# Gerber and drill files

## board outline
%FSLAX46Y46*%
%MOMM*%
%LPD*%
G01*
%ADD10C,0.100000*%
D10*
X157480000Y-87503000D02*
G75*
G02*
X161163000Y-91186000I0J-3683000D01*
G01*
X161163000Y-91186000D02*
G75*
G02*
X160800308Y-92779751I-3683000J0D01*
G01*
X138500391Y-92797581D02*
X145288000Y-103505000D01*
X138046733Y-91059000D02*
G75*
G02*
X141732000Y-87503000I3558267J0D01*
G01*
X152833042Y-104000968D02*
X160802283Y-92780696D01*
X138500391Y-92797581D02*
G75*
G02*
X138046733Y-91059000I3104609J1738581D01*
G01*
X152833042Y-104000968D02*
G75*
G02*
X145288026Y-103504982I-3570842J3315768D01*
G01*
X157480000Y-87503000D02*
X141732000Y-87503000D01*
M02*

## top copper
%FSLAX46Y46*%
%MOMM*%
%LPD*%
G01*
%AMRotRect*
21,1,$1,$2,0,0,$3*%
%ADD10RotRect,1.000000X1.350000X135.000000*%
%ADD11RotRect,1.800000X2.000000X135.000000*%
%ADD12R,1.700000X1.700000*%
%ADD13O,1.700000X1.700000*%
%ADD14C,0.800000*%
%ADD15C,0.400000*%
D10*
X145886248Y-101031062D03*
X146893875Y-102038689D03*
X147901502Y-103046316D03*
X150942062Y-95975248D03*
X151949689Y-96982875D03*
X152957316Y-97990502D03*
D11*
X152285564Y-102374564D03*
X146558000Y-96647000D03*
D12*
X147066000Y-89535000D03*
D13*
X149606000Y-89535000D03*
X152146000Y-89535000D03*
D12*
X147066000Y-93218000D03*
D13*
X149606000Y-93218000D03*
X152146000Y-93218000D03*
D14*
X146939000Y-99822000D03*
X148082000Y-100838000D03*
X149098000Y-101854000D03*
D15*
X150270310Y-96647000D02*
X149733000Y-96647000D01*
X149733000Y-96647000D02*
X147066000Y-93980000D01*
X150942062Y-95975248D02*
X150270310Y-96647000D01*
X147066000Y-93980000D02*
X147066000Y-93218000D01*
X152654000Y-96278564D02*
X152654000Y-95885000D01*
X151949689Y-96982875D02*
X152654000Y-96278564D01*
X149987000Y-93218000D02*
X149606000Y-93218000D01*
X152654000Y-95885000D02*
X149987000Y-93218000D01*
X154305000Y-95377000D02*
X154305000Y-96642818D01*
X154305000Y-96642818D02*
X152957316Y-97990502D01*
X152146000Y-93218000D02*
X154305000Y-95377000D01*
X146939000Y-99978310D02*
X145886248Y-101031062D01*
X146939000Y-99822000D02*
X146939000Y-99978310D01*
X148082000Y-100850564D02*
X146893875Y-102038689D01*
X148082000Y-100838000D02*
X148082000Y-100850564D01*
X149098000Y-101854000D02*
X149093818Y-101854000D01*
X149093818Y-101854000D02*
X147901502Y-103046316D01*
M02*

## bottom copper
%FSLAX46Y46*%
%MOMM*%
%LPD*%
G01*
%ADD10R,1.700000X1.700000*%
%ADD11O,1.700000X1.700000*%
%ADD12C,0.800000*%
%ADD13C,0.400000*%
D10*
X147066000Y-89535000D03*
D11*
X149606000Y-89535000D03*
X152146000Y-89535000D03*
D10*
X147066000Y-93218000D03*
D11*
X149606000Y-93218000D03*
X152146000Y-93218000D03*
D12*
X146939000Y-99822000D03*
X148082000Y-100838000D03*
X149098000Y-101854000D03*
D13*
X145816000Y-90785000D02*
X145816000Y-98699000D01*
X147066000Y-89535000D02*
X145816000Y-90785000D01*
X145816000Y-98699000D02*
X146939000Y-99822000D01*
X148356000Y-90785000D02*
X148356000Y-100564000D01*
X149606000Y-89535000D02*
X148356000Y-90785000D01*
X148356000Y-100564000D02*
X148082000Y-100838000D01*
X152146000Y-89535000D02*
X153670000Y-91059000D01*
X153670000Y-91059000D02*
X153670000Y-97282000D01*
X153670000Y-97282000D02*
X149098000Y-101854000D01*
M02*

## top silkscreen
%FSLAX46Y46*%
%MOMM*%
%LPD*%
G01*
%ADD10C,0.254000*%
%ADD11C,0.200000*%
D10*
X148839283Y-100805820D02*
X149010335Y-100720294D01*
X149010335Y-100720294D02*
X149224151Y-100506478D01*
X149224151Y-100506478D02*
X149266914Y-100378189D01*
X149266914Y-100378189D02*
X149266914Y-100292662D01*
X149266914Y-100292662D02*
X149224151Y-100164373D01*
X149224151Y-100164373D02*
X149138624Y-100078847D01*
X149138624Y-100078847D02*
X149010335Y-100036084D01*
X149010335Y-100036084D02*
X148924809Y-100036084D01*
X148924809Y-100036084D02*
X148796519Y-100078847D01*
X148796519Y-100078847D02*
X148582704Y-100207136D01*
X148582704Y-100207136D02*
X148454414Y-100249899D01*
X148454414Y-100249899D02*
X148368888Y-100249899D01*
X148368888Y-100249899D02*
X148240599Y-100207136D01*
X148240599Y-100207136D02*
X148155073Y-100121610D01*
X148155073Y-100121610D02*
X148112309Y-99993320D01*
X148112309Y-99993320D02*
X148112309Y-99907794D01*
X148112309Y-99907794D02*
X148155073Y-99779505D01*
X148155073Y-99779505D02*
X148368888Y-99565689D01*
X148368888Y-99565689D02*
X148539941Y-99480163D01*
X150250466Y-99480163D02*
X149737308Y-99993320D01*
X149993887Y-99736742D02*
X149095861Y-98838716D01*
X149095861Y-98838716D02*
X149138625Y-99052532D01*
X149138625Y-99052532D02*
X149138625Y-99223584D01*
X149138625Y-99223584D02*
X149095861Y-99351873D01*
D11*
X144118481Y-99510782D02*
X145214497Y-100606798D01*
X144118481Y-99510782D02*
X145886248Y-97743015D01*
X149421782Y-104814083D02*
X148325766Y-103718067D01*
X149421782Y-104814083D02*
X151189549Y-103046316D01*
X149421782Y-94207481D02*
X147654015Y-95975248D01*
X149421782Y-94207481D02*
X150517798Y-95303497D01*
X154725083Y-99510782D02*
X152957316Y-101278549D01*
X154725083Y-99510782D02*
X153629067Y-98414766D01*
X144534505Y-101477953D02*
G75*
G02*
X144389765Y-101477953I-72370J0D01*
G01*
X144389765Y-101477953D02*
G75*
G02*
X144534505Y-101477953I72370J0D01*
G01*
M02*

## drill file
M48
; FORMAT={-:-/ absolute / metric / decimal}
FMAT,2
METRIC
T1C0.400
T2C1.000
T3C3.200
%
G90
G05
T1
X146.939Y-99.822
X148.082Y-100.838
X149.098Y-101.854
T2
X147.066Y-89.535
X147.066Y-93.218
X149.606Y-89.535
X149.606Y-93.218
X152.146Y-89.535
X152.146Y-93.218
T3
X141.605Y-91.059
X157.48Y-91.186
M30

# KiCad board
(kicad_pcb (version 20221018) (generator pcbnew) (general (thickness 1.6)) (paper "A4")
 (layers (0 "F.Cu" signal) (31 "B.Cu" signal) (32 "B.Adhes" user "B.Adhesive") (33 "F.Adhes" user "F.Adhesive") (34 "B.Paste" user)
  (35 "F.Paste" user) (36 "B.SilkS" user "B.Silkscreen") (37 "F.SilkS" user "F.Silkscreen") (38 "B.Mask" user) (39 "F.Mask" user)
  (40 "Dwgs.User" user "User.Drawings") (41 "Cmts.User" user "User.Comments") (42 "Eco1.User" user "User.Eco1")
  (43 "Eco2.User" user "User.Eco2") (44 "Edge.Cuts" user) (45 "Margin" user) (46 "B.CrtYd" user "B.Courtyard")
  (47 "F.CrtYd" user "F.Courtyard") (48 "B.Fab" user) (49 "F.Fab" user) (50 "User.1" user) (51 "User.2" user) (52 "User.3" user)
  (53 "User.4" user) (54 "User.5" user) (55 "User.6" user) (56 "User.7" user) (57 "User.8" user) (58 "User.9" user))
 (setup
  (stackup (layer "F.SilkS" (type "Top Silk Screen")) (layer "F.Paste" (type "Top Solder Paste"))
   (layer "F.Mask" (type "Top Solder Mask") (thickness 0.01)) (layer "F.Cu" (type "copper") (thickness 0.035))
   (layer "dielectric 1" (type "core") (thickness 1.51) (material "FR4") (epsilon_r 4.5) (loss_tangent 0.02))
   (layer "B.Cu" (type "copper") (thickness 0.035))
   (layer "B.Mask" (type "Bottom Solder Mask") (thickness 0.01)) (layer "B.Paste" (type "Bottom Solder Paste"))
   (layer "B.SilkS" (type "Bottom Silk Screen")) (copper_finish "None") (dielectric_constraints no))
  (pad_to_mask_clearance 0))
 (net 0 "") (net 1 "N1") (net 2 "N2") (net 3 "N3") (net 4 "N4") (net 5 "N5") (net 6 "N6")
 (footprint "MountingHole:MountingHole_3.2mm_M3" (layer "F.Cu") (at 141.605 91.059)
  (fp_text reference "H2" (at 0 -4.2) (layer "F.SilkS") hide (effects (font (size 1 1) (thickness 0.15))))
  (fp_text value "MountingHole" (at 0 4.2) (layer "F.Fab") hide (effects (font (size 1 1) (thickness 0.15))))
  (pad "" np_thru_hole circle (at 0 0) (size 3.2 3.2) (drill 3.2) (layers "*.Cu" "*.Mask")))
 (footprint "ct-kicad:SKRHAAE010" (layer "F.Cu") (at 149.421782 99.510782 45)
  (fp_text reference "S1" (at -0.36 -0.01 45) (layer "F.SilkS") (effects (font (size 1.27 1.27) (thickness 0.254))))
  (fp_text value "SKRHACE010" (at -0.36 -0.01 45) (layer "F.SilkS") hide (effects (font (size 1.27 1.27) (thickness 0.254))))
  (fp_line (start -3.75 -3.75) (end -3.75 -2.2) (stroke (width 0.2) (type solid)) (layer "F.SilkS"))
  (fp_line (start -3.75 -3.75) (end -1.25 -3.75) (stroke (width 0.2) (type solid)) (layer "F.SilkS"))
  (fp_line (start -3.75 3.75) (end -3.75 2.2) (stroke (width 0.2) (type solid)) (layer "F.SilkS"))
  (fp_line (start -3.75 3.75) (end -1.25 3.75) (stroke (width 0.2) (type solid)) (layer "F.SilkS"))
  (fp_line (start 3.75 -3.75) (end 1.25 -3.75) (stroke (width 0.2) (type solid)) (layer "F.SilkS"))
  (fp_line (start 3.75 -3.75) (end 3.75 -2.2) (stroke (width 0.2) (type solid)) (layer "F.SilkS"))
  (fp_line (start 3.75 3.75) (end 1.25 3.75) (stroke (width 0.2) (type solid)) (layer "F.SilkS"))
  (fp_line (start 3.75 3.75) (end 3.75 2.2) (stroke (width 0.2) (type solid)) (layer "F.SilkS"))
  (fp_circle (center -4.898 -2.116) (end -4.898 -2.04363) (stroke (width 0.2) (type solid)) (fill none) (layer "F.SilkS"))
  (pad "1" smd rect (at -3.575 -1.425 135) (size 1 1.35) (layers "F.Cu" "F.Paste" "F.Mask") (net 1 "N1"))
  (pad "2" smd rect (at -3.575 0 135) (size 1 1.35) (layers "F.Cu" "F.Paste" "F.Mask") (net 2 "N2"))
  (pad "3" smd rect (at -3.575 1.425 135) (size 1 1.35) (layers "F.Cu" "F.Paste" "F.Mask") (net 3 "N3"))
  (pad "4" smd rect (at 3.575 -1.425 135) (size 1 1.35) (layers "F.Cu" "F.Paste" "F.Mask") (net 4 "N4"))
  (pad "5" smd rect (at 3.575 0 135) (size 1 1.35) (layers "F.Cu" "F.Paste" "F.Mask") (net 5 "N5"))
  (pad "6" smd rect (at 3.575 1.425 135) (size 1 1.35) (layers "F.Cu" "F.Paste" "F.Mask") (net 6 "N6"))
  (pad "7" smd rect (at 0 4.05 135) (size 1.8 2) (layers "F.Cu" "F.Paste" "F.Mask"))
  (pad "8" smd rect (at 0 -4.05 135) (size 1.8 2) (layers "F.Cu" "F.Paste" "F.Mask")))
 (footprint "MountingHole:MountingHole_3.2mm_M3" (layer "F.Cu") (at 157.48 91.186 90)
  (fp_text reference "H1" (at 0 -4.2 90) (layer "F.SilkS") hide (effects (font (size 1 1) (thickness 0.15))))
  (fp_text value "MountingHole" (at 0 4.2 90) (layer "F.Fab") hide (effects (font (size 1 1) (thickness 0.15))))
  (pad "" np_thru_hole circle (at 0 0 90) (size 3.2 3.2) (drill 3.2) (layers "*.Cu" "*.Mask")))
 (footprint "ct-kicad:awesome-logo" (layer "B.Cu") (at 150.495 98.933 180)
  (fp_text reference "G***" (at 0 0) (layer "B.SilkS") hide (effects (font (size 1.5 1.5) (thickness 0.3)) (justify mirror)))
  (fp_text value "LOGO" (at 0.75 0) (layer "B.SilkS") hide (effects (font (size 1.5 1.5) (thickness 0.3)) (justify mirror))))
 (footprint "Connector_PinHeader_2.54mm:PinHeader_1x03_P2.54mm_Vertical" (layer "B.Cu") (at 147.066 89.535 -90)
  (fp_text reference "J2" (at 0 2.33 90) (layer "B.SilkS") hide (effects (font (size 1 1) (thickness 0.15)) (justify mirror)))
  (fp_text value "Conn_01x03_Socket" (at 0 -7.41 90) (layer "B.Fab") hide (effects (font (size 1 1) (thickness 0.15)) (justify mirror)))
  (pad "1" thru_hole rect (at 0 0 270) (size 1.7 1.7) (drill 1) (layers "*.Cu" "*.Mask") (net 1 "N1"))
  (pad "2" thru_hole oval (at 0 -2.54 270) (size 1.7 1.7) (drill 1) (layers "*.Cu" "*.Mask") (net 2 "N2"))
  (pad "3" thru_hole oval (at 0 -5.08 270) (size 1.7 1.7) (drill 1) (layers "*.Cu" "*.Mask") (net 3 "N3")))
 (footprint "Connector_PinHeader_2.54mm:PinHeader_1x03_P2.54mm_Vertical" (layer "B.Cu") (at 147.066 93.218 -90)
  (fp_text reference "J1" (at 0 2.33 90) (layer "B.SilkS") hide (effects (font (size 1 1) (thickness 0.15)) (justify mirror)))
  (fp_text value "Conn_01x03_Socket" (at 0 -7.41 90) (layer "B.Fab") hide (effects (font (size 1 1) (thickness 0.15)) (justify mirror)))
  (pad "1" thru_hole rect (at 0 0 270) (size 1.7 1.7) (drill 1) (layers "*.Cu" "*.Mask") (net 4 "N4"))
  (pad "2" thru_hole oval (at 0 -2.54 270) (size 1.7 1.7) (drill 1) (layers "*.Cu" "*.Mask") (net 5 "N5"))
  (pad "3" thru_hole oval (at 0 -5.08 270) (size 1.7 1.7) (drill 1) (layers "*.Cu" "*.Mask") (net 6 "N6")))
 (gr_arc (start 157.48 87.503) (mid 160.084274 88.581726) (end 161.163 91.186) (stroke (width 0.1) (type default)) (layer "Edge.Cuts"))
 (gr_arc (start 161.163 91.186) (mid 161.071183 92.00325) (end 160.800308 92.779751) (stroke (width 0.1) (type default)) (layer "Edge.Cuts"))
 (gr_line (start 138.500391 92.797581) (end 145.288 103.505) (stroke (width 0.1) (type default)) (layer "Edge.Cuts"))
 (gr_arc (start 138.046733 91.059) (mid 139.134235 88.498418) (end 141.732 87.503) (stroke (width 0.1) (type default)) (layer "Edge.Cuts"))
 (gr_line (start 152.833042 104.000968) (end 160.802283 92.780696) (stroke (width 0.1) (type default)) (layer "Edge.Cuts"))
 (gr_arc (start 138.500391 92.797581) (mid 138.162015 91.957397) (end 138.046733 91.059) (stroke (width 0.1) (type default))
  (layer "Edge.Cuts"))
 (gr_arc (start 152.833042 104.000968) (mid 148.942552 105.547617) (end 145.288 103.505) (stroke (width 0.1) (type default))
  (layer "Edge.Cuts"))
 (gr_line (start 157.48 87.503) (end 141.732 87.503) (stroke (width 0.1) (type default)) (layer "Edge.Cuts"))
 (segment (start 150.27031 96.647) (end 149.733 96.647) (width 0.4) (layer "F.Cu") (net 4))
 (segment (start 149.733 96.647) (end 147.066 93.98) (width 0.4) (layer "F.Cu") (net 4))
 (segment (start 150.942062 95.975248) (end 150.27031 96.647) (width 0.4) (layer "F.Cu") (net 4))
 (segment (start 147.066 93.98) (end 147.066 93.218) (width 0.4) (layer "F.Cu") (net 4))
 (segment (start 152.654 96.278564) (end 152.654 95.885) (width 0.4) (layer "F.Cu") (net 5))
 (segment (start 151.949689 96.982875) (end 152.654 96.278564) (width 0.4) (layer "F.Cu") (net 5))
 (segment (start 149.987 93.218) (end 149.606 93.218) (width 0.4) (layer "F.Cu") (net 5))
 (segment (start 152.654 95.885) (end 149.987 93.218) (width 0.4) (layer "F.Cu") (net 5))
 (segment (start 154.305 95.377) (end 154.305 96.642818) (width 0.4) (layer "F.Cu") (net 6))
 (segment (start 154.305 96.642818) (end 152.957316 97.990502) (width 0.4) (layer "F.Cu") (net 6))
 (segment (start 152.146 93.218) (end 154.305 95.377) (width 0.4) (layer "F.Cu") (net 6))
 (segment (start 146.939 99.97831) (end 145.886248 101.031062) (width 0.4) (layer "F.Cu") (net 1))
 (segment (start 146.939 99.822) (end 146.939 99.97831) (width 0.4) (layer "F.Cu") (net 1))
 (via (at 146.939 99.822) (size 0.8) (drill 0.4) (layers "F.Cu" "B.Cu") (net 1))
 (segment (start 145.816 90.785) (end 145.816 98.699) (width 0.4) (layer "B.Cu") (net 1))
 (segment (start 147.066 89.535) (end 145.816 90.785) (width 0.4) (layer "B.Cu") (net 1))
 (segment (start 145.816 98.699) (end 146.939 99.822) (width 0.4) (layer "B.Cu") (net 1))
 (segment (start 148.082 100.850564) (end 146.893875 102.038689) (width 0.4) (layer "F.Cu") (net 2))
 (segment (start 148.082 100.838) (end 148.082 100.850564) (width 0.4) (layer "F.Cu") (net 2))
 (via (at 148.082 100.838) (size 0.8) (drill 0.4) (layers "F.Cu" "B.Cu") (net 2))
 (segment (start 148.356 90.785) (end 148.356 100.564) (width 0.4) (layer "B.Cu") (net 2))
 (segment (start 149.606 89.535) (end 148.356 90.785) (width 0.4) (layer "B.Cu") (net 2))
 (segment (start 148.356 100.564) (end 148.082 100.838) (width 0.4) (layer "B.Cu") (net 2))
 (segment (start 149.098 101.854) (end 149.093818 101.854) (width 0.4) (layer "F.Cu") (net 3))
 (segment (start 149.093818 101.854) (end 147.901502 103.046316) (width 0.4) (layer "F.Cu") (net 3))
 (via (at 149.098 101.854) (size 0.8) (drill 0.4) (layers "F.Cu" "B.Cu") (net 3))
 (segment (start 152.146 89.535) (end 153.67 91.059) (width 0.4) (layer "B.Cu") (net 3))
 (segment (start 153.67 91.059) (end 153.67 97.282) (width 0.4) (layer "B.Cu") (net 3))
 (segment (start 153.67 97.282) (end 149.098 101.854) (width 0.4) (layer "B.Cu") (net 3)))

